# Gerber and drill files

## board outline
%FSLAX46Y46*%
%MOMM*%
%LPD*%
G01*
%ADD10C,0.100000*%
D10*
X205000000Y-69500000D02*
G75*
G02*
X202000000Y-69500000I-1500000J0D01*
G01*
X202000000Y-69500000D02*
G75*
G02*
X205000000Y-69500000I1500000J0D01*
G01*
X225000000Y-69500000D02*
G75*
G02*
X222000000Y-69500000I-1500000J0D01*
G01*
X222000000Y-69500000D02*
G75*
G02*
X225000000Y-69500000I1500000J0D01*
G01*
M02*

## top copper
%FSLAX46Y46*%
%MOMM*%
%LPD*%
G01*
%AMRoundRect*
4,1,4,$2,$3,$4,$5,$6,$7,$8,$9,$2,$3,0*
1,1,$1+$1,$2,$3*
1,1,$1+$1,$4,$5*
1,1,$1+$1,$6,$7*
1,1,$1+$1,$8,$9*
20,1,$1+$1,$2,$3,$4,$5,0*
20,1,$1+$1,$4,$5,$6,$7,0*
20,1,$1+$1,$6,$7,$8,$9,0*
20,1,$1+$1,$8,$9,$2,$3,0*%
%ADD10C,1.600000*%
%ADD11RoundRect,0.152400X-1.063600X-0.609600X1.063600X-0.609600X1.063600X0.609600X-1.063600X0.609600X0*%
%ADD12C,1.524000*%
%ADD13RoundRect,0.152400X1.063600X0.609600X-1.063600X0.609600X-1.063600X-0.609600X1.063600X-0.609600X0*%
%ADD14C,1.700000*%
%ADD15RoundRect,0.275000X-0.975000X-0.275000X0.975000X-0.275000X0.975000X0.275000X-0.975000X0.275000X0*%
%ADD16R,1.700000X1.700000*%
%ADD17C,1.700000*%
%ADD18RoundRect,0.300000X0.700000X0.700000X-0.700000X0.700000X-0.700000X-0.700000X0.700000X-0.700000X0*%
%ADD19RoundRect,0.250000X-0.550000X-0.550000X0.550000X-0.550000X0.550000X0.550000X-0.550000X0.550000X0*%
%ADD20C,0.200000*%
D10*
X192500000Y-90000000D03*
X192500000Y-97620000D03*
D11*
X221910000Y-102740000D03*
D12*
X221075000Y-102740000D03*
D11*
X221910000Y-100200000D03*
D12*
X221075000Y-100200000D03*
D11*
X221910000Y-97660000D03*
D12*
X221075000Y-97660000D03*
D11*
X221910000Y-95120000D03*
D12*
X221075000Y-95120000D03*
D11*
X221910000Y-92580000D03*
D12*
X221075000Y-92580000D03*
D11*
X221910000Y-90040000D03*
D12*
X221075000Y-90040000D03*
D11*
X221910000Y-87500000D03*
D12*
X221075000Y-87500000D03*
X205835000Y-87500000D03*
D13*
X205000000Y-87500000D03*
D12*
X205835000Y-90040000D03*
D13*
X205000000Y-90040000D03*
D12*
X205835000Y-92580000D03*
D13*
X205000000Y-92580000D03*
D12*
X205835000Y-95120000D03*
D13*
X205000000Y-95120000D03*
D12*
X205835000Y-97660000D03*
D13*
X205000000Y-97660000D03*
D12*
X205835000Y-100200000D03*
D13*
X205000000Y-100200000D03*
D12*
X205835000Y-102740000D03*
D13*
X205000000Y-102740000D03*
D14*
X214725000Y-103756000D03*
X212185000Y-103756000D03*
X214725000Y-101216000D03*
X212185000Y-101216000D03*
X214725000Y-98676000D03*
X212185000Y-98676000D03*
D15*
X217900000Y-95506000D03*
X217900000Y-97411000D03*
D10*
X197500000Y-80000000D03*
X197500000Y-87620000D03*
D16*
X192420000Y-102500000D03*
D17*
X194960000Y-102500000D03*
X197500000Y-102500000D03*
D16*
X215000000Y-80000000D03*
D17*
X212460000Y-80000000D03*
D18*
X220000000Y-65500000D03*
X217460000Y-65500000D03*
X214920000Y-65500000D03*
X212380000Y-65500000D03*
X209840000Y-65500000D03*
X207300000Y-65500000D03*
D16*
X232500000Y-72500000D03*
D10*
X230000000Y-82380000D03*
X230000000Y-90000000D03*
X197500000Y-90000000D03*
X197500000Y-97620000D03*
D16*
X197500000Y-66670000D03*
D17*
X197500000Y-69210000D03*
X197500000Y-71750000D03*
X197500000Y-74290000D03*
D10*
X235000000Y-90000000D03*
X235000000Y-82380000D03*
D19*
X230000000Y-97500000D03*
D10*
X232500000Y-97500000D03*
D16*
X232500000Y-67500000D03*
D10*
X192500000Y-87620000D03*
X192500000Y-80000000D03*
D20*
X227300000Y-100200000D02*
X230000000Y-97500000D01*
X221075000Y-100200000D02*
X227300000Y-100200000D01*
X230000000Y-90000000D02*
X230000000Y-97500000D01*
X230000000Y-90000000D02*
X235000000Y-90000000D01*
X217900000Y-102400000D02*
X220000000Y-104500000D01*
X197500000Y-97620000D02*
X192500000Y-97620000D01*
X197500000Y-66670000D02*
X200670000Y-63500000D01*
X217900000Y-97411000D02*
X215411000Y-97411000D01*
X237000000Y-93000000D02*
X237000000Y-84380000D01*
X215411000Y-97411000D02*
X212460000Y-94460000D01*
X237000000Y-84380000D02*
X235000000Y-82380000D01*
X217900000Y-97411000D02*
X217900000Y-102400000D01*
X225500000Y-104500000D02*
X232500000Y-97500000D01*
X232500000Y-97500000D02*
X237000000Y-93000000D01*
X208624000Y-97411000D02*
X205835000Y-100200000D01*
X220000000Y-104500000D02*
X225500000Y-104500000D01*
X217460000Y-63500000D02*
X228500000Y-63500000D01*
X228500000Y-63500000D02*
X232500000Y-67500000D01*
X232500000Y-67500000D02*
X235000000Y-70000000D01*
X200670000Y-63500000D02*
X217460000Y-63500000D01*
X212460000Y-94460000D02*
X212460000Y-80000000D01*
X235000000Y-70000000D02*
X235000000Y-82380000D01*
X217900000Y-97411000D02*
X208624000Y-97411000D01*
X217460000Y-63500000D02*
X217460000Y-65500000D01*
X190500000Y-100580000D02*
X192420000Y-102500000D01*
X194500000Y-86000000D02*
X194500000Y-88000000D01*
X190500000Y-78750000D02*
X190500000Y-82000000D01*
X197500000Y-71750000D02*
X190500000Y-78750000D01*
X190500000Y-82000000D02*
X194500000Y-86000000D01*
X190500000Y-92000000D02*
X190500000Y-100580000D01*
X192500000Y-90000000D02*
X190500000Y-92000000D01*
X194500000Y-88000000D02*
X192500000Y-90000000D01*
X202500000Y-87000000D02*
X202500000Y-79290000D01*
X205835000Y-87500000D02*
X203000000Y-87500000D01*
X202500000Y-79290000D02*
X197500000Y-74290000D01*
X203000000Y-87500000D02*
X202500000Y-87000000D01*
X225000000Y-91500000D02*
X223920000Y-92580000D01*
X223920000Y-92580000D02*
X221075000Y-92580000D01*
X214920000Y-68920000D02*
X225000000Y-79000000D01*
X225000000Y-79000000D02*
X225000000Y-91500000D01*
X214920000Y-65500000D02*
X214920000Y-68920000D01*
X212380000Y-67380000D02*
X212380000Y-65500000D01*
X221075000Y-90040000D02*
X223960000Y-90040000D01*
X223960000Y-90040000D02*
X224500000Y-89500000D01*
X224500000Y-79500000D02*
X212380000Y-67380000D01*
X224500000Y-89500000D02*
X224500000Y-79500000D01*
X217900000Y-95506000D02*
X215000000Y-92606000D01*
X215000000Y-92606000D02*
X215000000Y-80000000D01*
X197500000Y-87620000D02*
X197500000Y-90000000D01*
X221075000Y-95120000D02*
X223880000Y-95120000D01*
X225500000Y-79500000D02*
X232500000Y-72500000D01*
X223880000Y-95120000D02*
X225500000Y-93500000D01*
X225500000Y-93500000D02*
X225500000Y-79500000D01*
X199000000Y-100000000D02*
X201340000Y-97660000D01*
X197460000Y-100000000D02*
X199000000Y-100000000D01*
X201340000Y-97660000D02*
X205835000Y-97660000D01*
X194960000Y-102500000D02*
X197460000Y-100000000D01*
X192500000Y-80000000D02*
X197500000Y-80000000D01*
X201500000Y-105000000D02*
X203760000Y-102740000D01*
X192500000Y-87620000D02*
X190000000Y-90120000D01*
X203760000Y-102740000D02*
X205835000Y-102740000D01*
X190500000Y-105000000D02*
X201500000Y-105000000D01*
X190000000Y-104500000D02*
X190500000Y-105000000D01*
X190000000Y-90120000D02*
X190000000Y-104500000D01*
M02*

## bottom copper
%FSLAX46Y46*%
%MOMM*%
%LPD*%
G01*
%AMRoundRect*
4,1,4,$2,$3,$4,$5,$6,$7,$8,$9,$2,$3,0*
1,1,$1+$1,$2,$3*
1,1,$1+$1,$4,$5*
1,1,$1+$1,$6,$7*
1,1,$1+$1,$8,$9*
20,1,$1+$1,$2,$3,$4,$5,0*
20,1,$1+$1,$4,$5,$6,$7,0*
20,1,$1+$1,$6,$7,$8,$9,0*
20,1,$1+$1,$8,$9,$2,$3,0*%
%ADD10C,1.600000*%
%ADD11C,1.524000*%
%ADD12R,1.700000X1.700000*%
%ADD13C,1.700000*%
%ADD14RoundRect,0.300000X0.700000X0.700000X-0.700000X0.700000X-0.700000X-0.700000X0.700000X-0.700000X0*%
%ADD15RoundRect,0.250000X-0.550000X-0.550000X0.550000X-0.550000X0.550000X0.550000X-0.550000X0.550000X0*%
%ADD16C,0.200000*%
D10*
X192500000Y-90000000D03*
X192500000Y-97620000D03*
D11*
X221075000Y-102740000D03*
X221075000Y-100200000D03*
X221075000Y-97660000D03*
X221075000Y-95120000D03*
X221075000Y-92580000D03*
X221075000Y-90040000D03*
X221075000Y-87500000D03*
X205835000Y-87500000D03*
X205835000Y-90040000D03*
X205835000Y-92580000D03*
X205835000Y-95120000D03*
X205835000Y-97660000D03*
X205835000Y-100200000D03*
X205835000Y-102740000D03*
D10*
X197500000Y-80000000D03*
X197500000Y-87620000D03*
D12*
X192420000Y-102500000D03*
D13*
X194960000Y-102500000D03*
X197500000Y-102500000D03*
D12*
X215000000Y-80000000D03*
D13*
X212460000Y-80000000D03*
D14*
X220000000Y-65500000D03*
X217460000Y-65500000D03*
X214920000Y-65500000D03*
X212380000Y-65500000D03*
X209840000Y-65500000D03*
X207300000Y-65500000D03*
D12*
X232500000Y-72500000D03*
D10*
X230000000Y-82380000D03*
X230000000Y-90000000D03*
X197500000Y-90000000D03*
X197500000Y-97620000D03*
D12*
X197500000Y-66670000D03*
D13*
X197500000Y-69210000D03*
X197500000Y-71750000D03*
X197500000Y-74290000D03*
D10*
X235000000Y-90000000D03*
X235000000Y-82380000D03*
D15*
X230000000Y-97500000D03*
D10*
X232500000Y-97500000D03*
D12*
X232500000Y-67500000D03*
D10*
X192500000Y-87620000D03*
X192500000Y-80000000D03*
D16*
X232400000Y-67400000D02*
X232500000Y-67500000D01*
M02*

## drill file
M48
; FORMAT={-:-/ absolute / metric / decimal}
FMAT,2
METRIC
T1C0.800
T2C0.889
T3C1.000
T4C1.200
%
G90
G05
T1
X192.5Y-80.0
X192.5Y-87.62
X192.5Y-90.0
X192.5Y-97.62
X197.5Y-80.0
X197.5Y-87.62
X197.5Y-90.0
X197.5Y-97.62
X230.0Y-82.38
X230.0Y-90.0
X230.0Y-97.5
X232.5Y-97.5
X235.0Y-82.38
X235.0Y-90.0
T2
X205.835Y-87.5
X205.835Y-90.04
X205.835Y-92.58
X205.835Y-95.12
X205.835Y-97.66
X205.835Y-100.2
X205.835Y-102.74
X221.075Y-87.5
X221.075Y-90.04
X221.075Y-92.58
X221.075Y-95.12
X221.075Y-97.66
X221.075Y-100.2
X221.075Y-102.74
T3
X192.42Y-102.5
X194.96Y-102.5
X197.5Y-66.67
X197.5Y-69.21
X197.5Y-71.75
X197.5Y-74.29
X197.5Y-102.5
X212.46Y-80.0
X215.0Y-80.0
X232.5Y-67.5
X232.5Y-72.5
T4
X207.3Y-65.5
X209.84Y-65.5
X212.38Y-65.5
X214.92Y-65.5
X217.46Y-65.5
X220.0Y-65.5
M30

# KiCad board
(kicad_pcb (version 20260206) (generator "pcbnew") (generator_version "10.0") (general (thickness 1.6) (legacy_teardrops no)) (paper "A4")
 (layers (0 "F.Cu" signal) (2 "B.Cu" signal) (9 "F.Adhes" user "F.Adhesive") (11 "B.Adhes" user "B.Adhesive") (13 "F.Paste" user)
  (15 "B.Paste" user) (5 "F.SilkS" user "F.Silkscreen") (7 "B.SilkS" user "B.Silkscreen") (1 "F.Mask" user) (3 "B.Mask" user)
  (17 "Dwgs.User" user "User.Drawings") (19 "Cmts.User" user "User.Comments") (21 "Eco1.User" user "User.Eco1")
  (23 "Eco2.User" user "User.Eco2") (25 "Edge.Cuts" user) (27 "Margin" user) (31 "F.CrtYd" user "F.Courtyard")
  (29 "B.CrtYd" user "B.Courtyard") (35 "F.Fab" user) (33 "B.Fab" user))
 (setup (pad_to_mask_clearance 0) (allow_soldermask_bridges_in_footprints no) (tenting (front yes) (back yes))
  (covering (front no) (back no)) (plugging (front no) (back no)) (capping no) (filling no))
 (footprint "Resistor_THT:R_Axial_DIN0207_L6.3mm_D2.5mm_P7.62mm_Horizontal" (layer "F.Cu") (at 192.5 90 -90)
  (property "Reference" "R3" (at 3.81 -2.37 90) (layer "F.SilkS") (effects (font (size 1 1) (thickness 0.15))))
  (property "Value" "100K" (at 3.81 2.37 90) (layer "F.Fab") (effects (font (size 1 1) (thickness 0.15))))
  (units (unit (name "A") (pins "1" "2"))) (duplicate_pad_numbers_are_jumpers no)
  (pad "1" thru_hole circle (at 0 0 270) (size 1.6 1.6) (drill 0.8) (layers "*.Cu" "*.Mask") (remove_unused_layers no) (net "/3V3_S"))
  (pad "2" thru_hole circle (at 7.62 0 270) (size 1.6 1.6) (drill 0.8) (layers "*.Cu" "*.Mask") (remove_unused_layers no) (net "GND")))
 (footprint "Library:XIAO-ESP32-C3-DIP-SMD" (layer "F.Cu") (at 213.455 95.12 -90)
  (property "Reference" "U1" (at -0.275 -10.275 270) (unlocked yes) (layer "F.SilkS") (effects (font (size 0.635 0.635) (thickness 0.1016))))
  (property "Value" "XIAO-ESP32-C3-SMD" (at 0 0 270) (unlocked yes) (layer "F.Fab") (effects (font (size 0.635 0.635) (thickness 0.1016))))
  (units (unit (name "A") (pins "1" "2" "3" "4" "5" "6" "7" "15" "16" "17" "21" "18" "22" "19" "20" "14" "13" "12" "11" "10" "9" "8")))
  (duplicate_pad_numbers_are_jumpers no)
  (pad "1" smd roundrect (at 7.62 -8.455) (size 2.432 1.524) (layers "F.Cu" "F.Mask") (roundrect_rratio 0.1)
   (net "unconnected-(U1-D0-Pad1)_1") (thermal_bridge_angle 45))
  (pad "1" thru_hole circle (at 7.62 -7.62) (size 1.524 1.524) (drill 0.889) (layers "*.Cu" "*.Mask") (remove_unused_layers no)
   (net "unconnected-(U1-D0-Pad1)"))
  (pad "2" smd roundrect (at 5.08 -8.455) (size 2.432 1.524) (layers "F.Cu" "F.Mask") (roundrect_rratio 0.1) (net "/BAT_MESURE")
   (thermal_bridge_angle 45))
  (pad "2" thru_hole circle (at 5.08 -7.62) (size 1.524 1.524) (drill 0.889) (layers "*.Cu" "*.Mask") (remove_unused_layers no)
   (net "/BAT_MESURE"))
  (pad "3" smd roundrect (at 2.54 -8.455) (size 2.432 1.524) (layers "F.Cu" "F.Mask") (roundrect_rratio 0.1) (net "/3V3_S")
   (thermal_bridge_angle 45))
  (pad "3" thru_hole circle (at 2.54 -7.62) (size 1.524 1.524) (drill 0.889) (layers "*.Cu" "*.Mask") (remove_unused_layers no)
   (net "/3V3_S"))
  (pad "4" smd roundrect (at 0 -8.455) (size 2.432 1.524) (layers "F.Cu" "F.Mask") (roundrect_rratio 0.1) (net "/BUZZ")
   (thermal_bridge_angle 45))
  (pad "4" thru_hole circle (at 0 -7.62) (size 1.524 1.524) (drill 0.889) (layers "*.Cu" "*.Mask") (remove_unused_layers no) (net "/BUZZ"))
  (pad "5" smd roundrect (at -2.54 -8.455) (size 2.432 1.524) (layers "F.Cu" "F.Mask") (roundrect_rratio 0.1) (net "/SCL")
   (thermal_bridge_angle 45))
  (pad "5" thru_hole circle (at -2.54 -7.62) (size 1.524 1.524) (drill 0.889) (layers "*.Cu" "*.Mask") (remove_unused_layers no)
   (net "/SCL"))
  (pad "6" smd roundrect (at -5.08 -8.455) (size 2.432 1.524) (layers "F.Cu" "F.Mask") (roundrect_rratio 0.1) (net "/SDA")
   (thermal_bridge_angle 45))
  (pad "6" thru_hole circle (at -5.08 -7.62) (size 1.524 1.524) (drill 0.889) (layers "*.Cu" "*.Mask") (remove_unused_layers no)
   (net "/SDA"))
  (pad "7" smd roundrect (at -7.62 -8.455) (size 2.432 1.524) (layers "F.Cu" "F.Mask") (roundrect_rratio 0.1)
   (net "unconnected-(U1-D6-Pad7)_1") (thermal_bridge_angle 45))
  (pad "7" thru_hole circle (at -7.62 -7.62) (size 1.524 1.524) (drill 0.889) (layers "*.Cu" "*.Mask") (remove_unused_layers no)
   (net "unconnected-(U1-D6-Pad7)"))
  (pad "8" thru_hole circle (at -7.62 7.62 180) (size 1.524 1.524) (drill 0.889) (layers "*.Cu" "*.Mask") (remove_unused_layers no)
   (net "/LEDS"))
  (pad "8" smd roundrect (at -7.62 8.455 180) (size 2.432 1.524) (layers "F.Cu" "F.Mask") (roundrect_rratio 0.1) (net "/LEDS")
   (thermal_bridge_angle 45))
  (pad "9" thru_hole circle (at -5.08 7.62 180) (size 1.524 1.524) (drill 0.889) (layers "*.Cu" "*.Mask") (remove_unused_layers no)
   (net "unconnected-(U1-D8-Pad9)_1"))
  (pad "9" smd roundrect (at -5.08 8.455 180) (size 2.432 1.524) (layers "F.Cu" "F.Mask") (roundrect_rratio 0.1)
   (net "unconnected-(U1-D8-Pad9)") (thermal_bridge_angle 45))
  (pad "10" thru_hole circle (at -2.54 7.62 180) (size 1.524 1.524) (drill 0.889) (layers "*.Cu" "*.Mask") (remove_unused_layers no)
   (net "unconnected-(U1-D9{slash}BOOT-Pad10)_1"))
  (pad "10" smd roundrect (at -2.54 8.455 180) (size 2.432 1.524) (layers "F.Cu" "F.Mask") (roundrect_rratio 0.1)
   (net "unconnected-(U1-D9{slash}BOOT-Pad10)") (thermal_bridge_angle 45))
  (pad "11" thru_hole circle (at 0 7.62 180) (size 1.524 1.524) (drill 0.889) (layers "*.Cu" "*.Mask") (remove_unused_layers no)
   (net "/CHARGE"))
  (pad "11" smd roundrect (at 0 8.455 180) (size 2.432 1.524) (layers "F.Cu" "F.Mask") (roundrect_rratio 0.1) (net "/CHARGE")
   (thermal_bridge_angle 45))
  (pad "12" thru_hole circle (at 2.54 7.62 180) (size 1.524 1.524) (drill 0.889) (layers "*.Cu" "*.Mask") (remove_unused_layers no)
   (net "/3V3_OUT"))
  (pad "12" smd roundrect (at 2.54 8.455 180) (size 2.432 1.524) (layers "F.Cu" "F.Mask") (roundrect_rratio 0.1) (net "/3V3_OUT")
   (thermal_bridge_angle 45))
  (pad "13" thru_hole circle (at 5.08 7.62 180) (size 1.524 1.524) (drill 0.889) (layers "*.Cu" "*.Mask") (remove_unused_layers no)
   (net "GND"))
  (pad "13" smd roundrect (at 5.08 8.455 180) (size 2.432 1.524) (layers "F.Cu" "F.Mask") (roundrect_rratio 0.1) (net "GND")
   (thermal_bridge_angle 45))
  (pad "14" thru_hole circle (at 7.62 7.62 180) (size 1.524 1.524) (drill 0.889) (layers "*.Cu" "*.Mask") (remove_unused_layers no)
   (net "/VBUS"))
  (pad "14" smd roundrect (at 7.62 8.455 180) (size 2.432 1.524) (layers "F.Cu" "F.Mask") (roundrect_rratio 0.1) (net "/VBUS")
   (thermal_bridge_angle 45))
  (pad "15" smd circle (at 8.636 -1.27 180) (size 1.7 1.7) (layers "F.Cu" "F.Mask" "F.Paste") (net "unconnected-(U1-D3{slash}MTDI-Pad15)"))
  (pad "16" smd circle (at 8.636 1.27 180) (size 1.7 1.7) (layers "F.Cu" "F.Mask" "F.Paste") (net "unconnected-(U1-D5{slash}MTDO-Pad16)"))
  (pad "17" smd circle (at 6.096 -1.27 180) (size 1.7 1.7) (layers "F.Cu" "F.Mask" "F.Paste") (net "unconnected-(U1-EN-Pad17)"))
  (pad "18" smd circle (at 6.096 1.27 180) (size 1.7 1.7) (layers "F.Cu" "F.Mask" "F.Paste") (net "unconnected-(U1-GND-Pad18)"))
  (pad "19" smd circle (at 3.556 -1.27 180) (size 1.7 1.7) (layers "F.Cu" "F.Mask" "F.Paste") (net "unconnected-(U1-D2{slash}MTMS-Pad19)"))
  (pad "20" smd circle (at 3.556 1.27 180) (size 1.7 1.7) (layers "F.Cu" "F.Mask" "F.Paste") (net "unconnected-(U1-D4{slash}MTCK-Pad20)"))
  (pad "21" smd roundrect (at 0.386 -4.445) (size 2.5 1.1) (layers "F.Cu" "F.Mask" "F.Paste") (roundrect_rratio 0.25) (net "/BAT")
   (thermal_bridge_angle 45))
  (pad "22" smd roundrect (at 2.291 -4.445) (size 2.5 1.1) (layers "F.Cu" "F.Mask" "F.Paste") (roundrect_rratio 0.25) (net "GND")
   (thermal_bridge_angle 45)))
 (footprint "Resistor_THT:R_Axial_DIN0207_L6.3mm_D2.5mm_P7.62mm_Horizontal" (layer "F.Cu") (at 197.5 80 -90)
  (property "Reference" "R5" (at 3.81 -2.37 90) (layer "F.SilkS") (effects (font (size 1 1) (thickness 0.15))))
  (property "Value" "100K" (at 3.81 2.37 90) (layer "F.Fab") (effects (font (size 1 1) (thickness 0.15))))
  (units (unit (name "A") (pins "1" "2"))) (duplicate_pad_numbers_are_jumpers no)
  (pad "1" thru_hole circle (at 0 0 270) (size 1.6 1.6) (drill 0.8) (layers "*.Cu" "*.Mask") (remove_unused_layers no) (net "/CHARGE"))
  (pad "2" thru_hole circle (at 7.62 0 270) (size 1.6 1.6) (drill 0.8) (layers "*.Cu" "*.Mask") (remove_unused_layers no)
   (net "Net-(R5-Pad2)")))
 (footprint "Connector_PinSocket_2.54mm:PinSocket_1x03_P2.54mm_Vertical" (layer "F.Cu") (at 192.42 102.5 90)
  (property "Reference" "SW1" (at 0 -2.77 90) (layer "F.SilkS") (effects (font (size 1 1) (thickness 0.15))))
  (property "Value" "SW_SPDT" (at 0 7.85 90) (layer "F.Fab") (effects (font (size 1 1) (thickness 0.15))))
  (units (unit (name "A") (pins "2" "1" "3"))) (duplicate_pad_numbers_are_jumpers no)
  (pad "1" thru_hole rect (at 0 0 90) (size 1.7 1.7) (drill 1) (layers "*.Cu" "*.Mask") (remove_unused_layers no) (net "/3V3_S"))
  (pad "2" thru_hole circle (at 0 2.54 90) (size 1.7 1.7) (drill 1) (layers "*.Cu" "*.Mask") (remove_unused_layers no) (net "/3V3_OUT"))
  (pad "3" thru_hole circle (at 0 5.08 90) (size 1.7 1.7) (drill 1) (layers "*.Cu" "*.Mask") (remove_unused_layers no)
   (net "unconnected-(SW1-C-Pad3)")))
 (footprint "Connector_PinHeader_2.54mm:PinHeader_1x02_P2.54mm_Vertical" (layer "F.Cu") (at 215 80 -90)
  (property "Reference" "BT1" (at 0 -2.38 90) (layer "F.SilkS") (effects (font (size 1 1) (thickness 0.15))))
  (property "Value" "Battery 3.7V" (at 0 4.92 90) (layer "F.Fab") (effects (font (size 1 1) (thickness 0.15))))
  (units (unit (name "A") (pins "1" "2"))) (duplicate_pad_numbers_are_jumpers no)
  (pad "1" thru_hole rect (at 0 0 270) (size 1.7 1.7) (drill 1) (layers "*.Cu" "*.Mask") (remove_unused_layers no) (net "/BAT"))
  (pad "2" thru_hole circle (at 0 2.54 270) (size 1.7 1.7) (drill 1) (layers "*.Cu" "*.Mask") (remove_unused_layers no) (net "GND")))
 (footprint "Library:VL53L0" (layer "F.Cu") (at 220 65.5 180)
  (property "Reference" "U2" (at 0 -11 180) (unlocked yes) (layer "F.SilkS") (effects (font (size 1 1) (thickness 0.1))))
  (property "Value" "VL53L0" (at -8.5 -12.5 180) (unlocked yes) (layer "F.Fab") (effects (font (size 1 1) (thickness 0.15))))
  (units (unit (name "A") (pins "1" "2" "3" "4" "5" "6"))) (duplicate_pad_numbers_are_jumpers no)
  (fp_circle (center 16.5 -4) (end 18 -4) (stroke (width 0.1) (type default)) (fill no) (layer "Edge.Cuts"))
  (fp_circle (center -3.5 -4) (end -2 -4) (stroke (width 0.1) (type default)) (fill no) (layer "Edge.Cuts"))
  (pad "1" thru_hole roundrect (at 0 0 180) (size 2 2) (drill 1.2) (layers "*.Cu" "*.Mask") (remove_unused_layers no)
   (roundrect_rratio 0.15) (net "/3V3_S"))
  (pad "2" thru_hole roundrect (at 2.54 0 180) (size 2 2) (drill 1.2) (layers "*.Cu" "*.Mask") (remove_unused_layers no)
   (roundrect_rratio 0.15) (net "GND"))
  (pad "3" thru_hole roundrect (at 5.08 0 180) (size 2 2) (drill 1.2) (layers "*.Cu" "*.Mask") (remove_unused_layers no)
   (roundrect_rratio 0.15) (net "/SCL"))
  (pad "4" thru_hole roundrect (at 7.62 0 180) (size 2 2) (drill 1.2) (layers "*.Cu" "*.Mask") (remove_unused_layers no)
   (roundrect_rratio 0.15) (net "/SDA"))
  (pad "5" thru_hole roundrect (at 10.16 0 180) (size 2 2) (drill 1.2) (layers "*.Cu" "*.Mask") (remove_unused_layers no)
   (roundrect_rratio 0.15) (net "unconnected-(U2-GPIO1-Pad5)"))
  (pad "6" thru_hole roundrect (at 12.7 0 180) (size 2 2) (drill 1.2) (layers "*.Cu" "*.Mask") (remove_unused_layers no)
   (roundrect_rratio 0.15) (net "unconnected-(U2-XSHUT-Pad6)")))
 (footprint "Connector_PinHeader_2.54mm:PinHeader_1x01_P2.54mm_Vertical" (layer "F.Cu") (at 232.5 72.5 90)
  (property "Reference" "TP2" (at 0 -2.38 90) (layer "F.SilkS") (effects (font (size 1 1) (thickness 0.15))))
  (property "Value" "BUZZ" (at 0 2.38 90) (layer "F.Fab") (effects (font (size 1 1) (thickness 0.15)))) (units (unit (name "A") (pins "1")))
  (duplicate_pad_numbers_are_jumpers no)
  (pad "1" thru_hole rect (at 0 0 90) (size 1.7 1.7) (drill 1) (layers "*.Cu" "*.Mask") (remove_unused_layers no) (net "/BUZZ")))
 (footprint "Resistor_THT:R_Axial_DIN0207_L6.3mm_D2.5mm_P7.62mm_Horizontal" (layer "F.Cu") (at 230 82.38 -90)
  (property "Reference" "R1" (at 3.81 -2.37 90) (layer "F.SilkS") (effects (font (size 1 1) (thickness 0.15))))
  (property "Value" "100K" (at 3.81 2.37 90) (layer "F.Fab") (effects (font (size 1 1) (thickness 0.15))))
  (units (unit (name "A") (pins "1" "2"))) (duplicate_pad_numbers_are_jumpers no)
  (pad "1" thru_hole circle (at 0 0 270) (size 1.6 1.6) (drill 0.8) (layers "*.Cu" "*.Mask") (remove_unused_layers no) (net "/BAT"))
  (pad "2" thru_hole circle (at 7.62 0 270) (size 1.6 1.6) (drill 0.8) (layers "*.Cu" "*.Mask") (remove_unused_layers no)
   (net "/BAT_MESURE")))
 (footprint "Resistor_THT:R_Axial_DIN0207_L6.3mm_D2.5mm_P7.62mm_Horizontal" (layer "F.Cu") (at 197.5 90 -90)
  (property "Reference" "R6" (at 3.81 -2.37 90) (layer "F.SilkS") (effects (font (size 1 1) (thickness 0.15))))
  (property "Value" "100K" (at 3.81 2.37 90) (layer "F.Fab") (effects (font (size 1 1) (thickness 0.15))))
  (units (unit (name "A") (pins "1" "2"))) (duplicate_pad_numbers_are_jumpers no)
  (pad "1" thru_hole circle (at 0 0 270) (size 1.6 1.6) (drill 0.8) (layers "*.Cu" "*.Mask") (remove_unused_layers no) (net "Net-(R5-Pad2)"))
  (pad "2" thru_hole circle (at 7.62 0 270) (size 1.6 1.6) (drill 0.8) (layers "*.Cu" "*.Mask") (remove_unused_layers no) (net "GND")))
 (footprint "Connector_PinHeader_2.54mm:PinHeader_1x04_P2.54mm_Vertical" (layer "F.Cu") (at 197.5 66.67)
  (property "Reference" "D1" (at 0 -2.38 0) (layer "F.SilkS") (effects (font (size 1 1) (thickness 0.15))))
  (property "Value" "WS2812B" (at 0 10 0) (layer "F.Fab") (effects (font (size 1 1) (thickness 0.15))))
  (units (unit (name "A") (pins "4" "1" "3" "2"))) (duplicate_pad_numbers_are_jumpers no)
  (pad "1" thru_hole rect (at 0 0) (size 1.7 1.7) (drill 1) (layers "*.Cu" "*.Mask") (remove_unused_layers no) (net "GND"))
  (pad "2" thru_hole circle (at 0 2.54) (size 1.7 1.7) (drill 1) (layers "*.Cu" "*.Mask") (remove_unused_layers no)
   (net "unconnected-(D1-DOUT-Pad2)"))
  (pad "3" thru_hole circle (at 0 5.08) (size 1.7 1.7) (drill 1) (layers "*.Cu" "*.Mask") (remove_unused_layers no) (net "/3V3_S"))
  (pad "4" thru_hole circle (at 0 7.62) (size 1.7 1.7) (drill 1) (layers "*.Cu" "*.Mask") (remove_unused_layers no) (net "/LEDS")))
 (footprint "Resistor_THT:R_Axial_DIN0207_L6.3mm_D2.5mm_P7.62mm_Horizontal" (layer "F.Cu") (at 235 90 90)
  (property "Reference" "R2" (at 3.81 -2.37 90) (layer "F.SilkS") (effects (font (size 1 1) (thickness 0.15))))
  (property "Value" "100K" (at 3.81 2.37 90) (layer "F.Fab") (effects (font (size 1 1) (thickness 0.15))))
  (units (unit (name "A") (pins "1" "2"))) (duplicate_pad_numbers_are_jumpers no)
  (pad "1" thru_hole circle (at 0 0 90) (size 1.6 1.6) (drill 0.8) (layers "*.Cu" "*.Mask") (remove_unused_layers no) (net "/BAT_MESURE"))
  (pad "2" thru_hole circle (at 7.62 0 90) (size 1.6 1.6) (drill 0.8) (layers "*.Cu" "*.Mask") (remove_unused_layers no) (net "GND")))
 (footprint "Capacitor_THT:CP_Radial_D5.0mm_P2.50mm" (layer "F.Cu") (at 230 97.5)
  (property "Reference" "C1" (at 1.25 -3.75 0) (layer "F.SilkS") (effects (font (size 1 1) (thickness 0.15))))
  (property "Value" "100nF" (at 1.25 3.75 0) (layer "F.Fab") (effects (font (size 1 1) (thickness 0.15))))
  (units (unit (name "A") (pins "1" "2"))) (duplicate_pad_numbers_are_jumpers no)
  (pad "1" thru_hole roundrect (at 0 0) (size 1.6 1.6) (drill 0.8) (layers "*.Cu" "*.Mask") (remove_unused_layers no)
   (roundrect_rratio 0.15625) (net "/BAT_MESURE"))
  (pad "2" thru_hole circle (at 2.5 0) (size 1.6 1.6) (drill 0.8) (layers "*.Cu" "*.Mask") (remove_unused_layers no) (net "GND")))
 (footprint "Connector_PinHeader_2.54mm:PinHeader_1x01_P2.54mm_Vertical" (layer "F.Cu") (at 232.5 67.5 90)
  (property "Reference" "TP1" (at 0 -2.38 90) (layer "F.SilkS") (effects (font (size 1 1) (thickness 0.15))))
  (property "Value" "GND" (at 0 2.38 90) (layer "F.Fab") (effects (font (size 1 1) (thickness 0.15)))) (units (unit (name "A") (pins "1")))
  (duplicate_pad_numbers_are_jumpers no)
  (pad "1" thru_hole rect (at 0 0 90) (size 1.7 1.7) (drill 1) (layers "*.Cu" "*.Mask") (remove_unused_layers no) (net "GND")))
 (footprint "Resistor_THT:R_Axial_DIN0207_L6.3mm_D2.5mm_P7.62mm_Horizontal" (layer "F.Cu") (at 192.5 87.62 90)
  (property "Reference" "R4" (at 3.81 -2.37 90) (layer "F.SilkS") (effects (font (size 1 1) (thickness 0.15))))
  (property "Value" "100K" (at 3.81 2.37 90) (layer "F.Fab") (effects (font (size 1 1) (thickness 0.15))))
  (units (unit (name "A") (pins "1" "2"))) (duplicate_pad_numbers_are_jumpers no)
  (pad "1" thru_hole circle (at 0 0 90) (size 1.6 1.6) (drill 0.8) (layers "*.Cu" "*.Mask") (remove_unused_layers no) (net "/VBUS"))
  (pad "2" thru_hole circle (at 7.62 0 90) (size 1.6 1.6) (drill 0.8) (layers "*.Cu" "*.Mask") (remove_unused_layers no) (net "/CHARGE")))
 (segment (start 227.3 100.2) (end 230 97.5) (width 0.2) (layer "F.Cu") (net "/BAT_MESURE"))
 (segment (start 221.075 100.2) (end 227.3 100.2) (width 0.2) (layer "F.Cu") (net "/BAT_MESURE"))
 (segment (start 230 90) (end 230 97.5) (width 0.2) (layer "F.Cu") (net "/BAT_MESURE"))
 (segment (start 230 90) (end 235 90) (width 0.2) (layer "F.Cu") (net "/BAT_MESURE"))
 (segment (start 217.9 102.4) (end 220 104.5) (width 0.2) (layer "F.Cu") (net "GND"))
 (segment (start 197.5 97.62) (end 192.5 97.62) (width 0.2) (layer "F.Cu") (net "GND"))
 (segment (start 197.5 66.67) (end 200.67 63.5) (width 0.2) (layer "F.Cu") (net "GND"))
 (segment (start 217.9 97.411) (end 215.411 97.411) (width 0.2) (layer "F.Cu") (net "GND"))
 (segment (start 237 93) (end 237 84.38) (width 0.2) (layer "F.Cu") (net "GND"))
 (segment (start 215.411 97.411) (end 212.46 94.46) (width 0.2) (layer "F.Cu") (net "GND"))
 (segment (start 237 84.38) (end 235 82.38) (width 0.2) (layer "F.Cu") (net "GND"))
 (segment (start 217.9 97.411) (end 217.9 102.4) (width 0.2) (layer "F.Cu") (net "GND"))
 (segment (start 225.5 104.5) (end 232.5 97.5) (width 0.2) (layer "F.Cu") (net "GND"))
 (segment (start 232.5 97.5) (end 237 93) (width 0.2) (layer "F.Cu") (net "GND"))
 (segment (start 208.624 97.411) (end 205.835 100.2) (width 0.2) (layer "F.Cu") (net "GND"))
 (segment (start 220 104.5) (end 225.5 104.5) (width 0.2) (layer "F.Cu") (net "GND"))
 (segment (start 217.46 63.5) (end 228.5 63.5) (width 0.2) (layer "F.Cu") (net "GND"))
 (segment (start 228.5 63.5) (end 232.5 67.5) (width 0.2) (layer "F.Cu") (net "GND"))
 (segment (start 232.5 67.5) (end 235 70) (width 0.2) (layer "F.Cu") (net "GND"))
 (segment (start 200.67 63.5) (end 217.46 63.5) (width 0.2) (layer "F.Cu") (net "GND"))
 (segment (start 212.46 94.46) (end 212.46 80) (width 0.2) (layer "F.Cu") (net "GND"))
 (segment (start 235 70) (end 235 82.38) (width 0.2) (layer "F.Cu") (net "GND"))
 (segment (start 217.9 97.411) (end 208.624 97.411) (width 0.2) (layer "F.Cu") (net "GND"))
 (segment (start 217.46 63.5) (end 217.46 65.5) (width 0.2) (layer "F.Cu") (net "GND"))
 (segment (start 232.4 67.4) (end 232.5 67.5) (width 0.2) (layer "B.Cu") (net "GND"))
 (segment (start 190.5 100.58) (end 192.42 102.5) (width 0.2) (layer "F.Cu") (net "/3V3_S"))
 (segment (start 194.5 86) (end 194.5 88) (width 0.2) (layer "F.Cu") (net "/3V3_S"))
 (segment (start 190.5 78.75) (end 190.5 82) (width 0.2) (layer "F.Cu") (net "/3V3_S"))
 (segment (start 197.5 71.75) (end 190.5 78.75) (width 0.2) (layer "F.Cu") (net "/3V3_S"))
 (segment (start 190.5 82) (end 194.5 86) (width 0.2) (layer "F.Cu") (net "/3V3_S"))
 (segment (start 190.5 92) (end 190.5 100.58) (width 0.2) (layer "F.Cu") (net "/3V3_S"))
 (segment (start 192.5 90) (end 190.5 92) (width 0.2) (layer "F.Cu") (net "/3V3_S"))
 (segment (start 194.5 88) (end 192.5 90) (width 0.2) (layer "F.Cu") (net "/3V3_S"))
 (segment (start 202.5 87) (end 202.5 79.29) (width 0.2) (layer "F.Cu") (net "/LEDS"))
 (segment (start 205.835 87.5) (end 203 87.5) (width 0.2) (layer "F.Cu") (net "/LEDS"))
 (segment (start 202.5 79.29) (end 197.5 74.29) (width 0.2) (layer "F.Cu") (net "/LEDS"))
 (segment (start 203 87.5) (end 202.5 87) (width 0.2) (layer "F.Cu") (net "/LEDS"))
 (segment (start 225 91.5) (end 223.92 92.58) (width 0.2) (layer "F.Cu") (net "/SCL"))
 (segment (start 223.92 92.58) (end 221.075 92.58) (width 0.2) (layer "F.Cu") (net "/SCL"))
 (segment (start 214.92 68.92) (end 225 79) (width 0.2) (layer "F.Cu") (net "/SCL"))
 (segment (start 225 79) (end 225 91.5) (width 0.2) (layer "F.Cu") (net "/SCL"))
 (segment (start 214.92 65.5) (end 214.92 68.92) (width 0.2) (layer "F.Cu") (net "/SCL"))
 (segment (start 212.38 67.38) (end 212.38 65.5) (width 0.2) (layer "F.Cu") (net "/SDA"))
 (segment (start 221.075 90.04) (end 223.96 90.04) (width 0.2) (layer "F.Cu") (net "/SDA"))
 (segment (start 223.96 90.04) (end 224.5 89.5) (width 0.2) (layer "F.Cu") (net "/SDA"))
 (segment (start 224.5 79.5) (end 212.38 67.38) (width 0.2) (layer "F.Cu") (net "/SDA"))
 (segment (start 224.5 89.5) (end 224.5 79.5) (width 0.2) (layer "F.Cu") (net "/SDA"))
 (segment (start 217.9 95.506) (end 215 92.606) (width 0.2) (layer "F.Cu") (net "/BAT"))
 (segment (start 215 92.606) (end 215 80) (width 0.2) (layer "F.Cu") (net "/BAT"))
 (segment (start 197.5 87.62) (end 197.5 90) (width 0.2) (layer "F.Cu") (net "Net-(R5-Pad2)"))
 (segment (start 221.075 95.12) (end 223.88 95.12) (width 0.2) (layer "F.Cu") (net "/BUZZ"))
 (segment (start 225.5 79.5) (end 232.5 72.5) (width 0.2) (layer "F.Cu") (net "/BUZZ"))
 (segment (start 223.88 95.12) (end 225.5 93.5) (width 0.2) (layer "F.Cu") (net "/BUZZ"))
 (segment (start 225.5 93.5) (end 225.5 79.5) (width 0.2) (layer "F.Cu") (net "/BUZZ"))
 (segment (start 199 100) (end 201.34 97.66) (width 0.2) (layer "F.Cu") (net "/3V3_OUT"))
 (segment (start 197.46 100) (end 199 100) (width 0.2) (layer "F.Cu") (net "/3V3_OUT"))
 (segment (start 201.34 97.66) (end 205.835 97.66) (width 0.2) (layer "F.Cu") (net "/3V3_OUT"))
 (segment (start 194.96 102.5) (end 197.46 100) (width 0.2) (layer "F.Cu") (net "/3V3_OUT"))
 (segment (start 192.5 80) (end 197.5 80) (width 0.2) (layer "F.Cu") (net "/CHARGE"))
 (segment (start 201.5 105) (end 203.76 102.74) (width 0.2) (layer "F.Cu") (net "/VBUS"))
 (segment (start 192.5 87.62) (end 190 90.12) (width 0.2) (layer "F.Cu") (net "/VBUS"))
 (segment (start 203.76 102.74) (end 205.835 102.74) (width 0.2) (layer "F.Cu") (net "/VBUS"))
 (segment (start 190.5 105) (end 201.5 105) (width 0.2) (layer "F.Cu") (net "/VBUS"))
 (segment (start 190 104.5) (end 190.5 105) (width 0.2) (layer "F.Cu") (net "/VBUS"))
 (segment (start 190 90.12) (end 190 104.5) (width 0.2) (layer "F.Cu") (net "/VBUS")))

